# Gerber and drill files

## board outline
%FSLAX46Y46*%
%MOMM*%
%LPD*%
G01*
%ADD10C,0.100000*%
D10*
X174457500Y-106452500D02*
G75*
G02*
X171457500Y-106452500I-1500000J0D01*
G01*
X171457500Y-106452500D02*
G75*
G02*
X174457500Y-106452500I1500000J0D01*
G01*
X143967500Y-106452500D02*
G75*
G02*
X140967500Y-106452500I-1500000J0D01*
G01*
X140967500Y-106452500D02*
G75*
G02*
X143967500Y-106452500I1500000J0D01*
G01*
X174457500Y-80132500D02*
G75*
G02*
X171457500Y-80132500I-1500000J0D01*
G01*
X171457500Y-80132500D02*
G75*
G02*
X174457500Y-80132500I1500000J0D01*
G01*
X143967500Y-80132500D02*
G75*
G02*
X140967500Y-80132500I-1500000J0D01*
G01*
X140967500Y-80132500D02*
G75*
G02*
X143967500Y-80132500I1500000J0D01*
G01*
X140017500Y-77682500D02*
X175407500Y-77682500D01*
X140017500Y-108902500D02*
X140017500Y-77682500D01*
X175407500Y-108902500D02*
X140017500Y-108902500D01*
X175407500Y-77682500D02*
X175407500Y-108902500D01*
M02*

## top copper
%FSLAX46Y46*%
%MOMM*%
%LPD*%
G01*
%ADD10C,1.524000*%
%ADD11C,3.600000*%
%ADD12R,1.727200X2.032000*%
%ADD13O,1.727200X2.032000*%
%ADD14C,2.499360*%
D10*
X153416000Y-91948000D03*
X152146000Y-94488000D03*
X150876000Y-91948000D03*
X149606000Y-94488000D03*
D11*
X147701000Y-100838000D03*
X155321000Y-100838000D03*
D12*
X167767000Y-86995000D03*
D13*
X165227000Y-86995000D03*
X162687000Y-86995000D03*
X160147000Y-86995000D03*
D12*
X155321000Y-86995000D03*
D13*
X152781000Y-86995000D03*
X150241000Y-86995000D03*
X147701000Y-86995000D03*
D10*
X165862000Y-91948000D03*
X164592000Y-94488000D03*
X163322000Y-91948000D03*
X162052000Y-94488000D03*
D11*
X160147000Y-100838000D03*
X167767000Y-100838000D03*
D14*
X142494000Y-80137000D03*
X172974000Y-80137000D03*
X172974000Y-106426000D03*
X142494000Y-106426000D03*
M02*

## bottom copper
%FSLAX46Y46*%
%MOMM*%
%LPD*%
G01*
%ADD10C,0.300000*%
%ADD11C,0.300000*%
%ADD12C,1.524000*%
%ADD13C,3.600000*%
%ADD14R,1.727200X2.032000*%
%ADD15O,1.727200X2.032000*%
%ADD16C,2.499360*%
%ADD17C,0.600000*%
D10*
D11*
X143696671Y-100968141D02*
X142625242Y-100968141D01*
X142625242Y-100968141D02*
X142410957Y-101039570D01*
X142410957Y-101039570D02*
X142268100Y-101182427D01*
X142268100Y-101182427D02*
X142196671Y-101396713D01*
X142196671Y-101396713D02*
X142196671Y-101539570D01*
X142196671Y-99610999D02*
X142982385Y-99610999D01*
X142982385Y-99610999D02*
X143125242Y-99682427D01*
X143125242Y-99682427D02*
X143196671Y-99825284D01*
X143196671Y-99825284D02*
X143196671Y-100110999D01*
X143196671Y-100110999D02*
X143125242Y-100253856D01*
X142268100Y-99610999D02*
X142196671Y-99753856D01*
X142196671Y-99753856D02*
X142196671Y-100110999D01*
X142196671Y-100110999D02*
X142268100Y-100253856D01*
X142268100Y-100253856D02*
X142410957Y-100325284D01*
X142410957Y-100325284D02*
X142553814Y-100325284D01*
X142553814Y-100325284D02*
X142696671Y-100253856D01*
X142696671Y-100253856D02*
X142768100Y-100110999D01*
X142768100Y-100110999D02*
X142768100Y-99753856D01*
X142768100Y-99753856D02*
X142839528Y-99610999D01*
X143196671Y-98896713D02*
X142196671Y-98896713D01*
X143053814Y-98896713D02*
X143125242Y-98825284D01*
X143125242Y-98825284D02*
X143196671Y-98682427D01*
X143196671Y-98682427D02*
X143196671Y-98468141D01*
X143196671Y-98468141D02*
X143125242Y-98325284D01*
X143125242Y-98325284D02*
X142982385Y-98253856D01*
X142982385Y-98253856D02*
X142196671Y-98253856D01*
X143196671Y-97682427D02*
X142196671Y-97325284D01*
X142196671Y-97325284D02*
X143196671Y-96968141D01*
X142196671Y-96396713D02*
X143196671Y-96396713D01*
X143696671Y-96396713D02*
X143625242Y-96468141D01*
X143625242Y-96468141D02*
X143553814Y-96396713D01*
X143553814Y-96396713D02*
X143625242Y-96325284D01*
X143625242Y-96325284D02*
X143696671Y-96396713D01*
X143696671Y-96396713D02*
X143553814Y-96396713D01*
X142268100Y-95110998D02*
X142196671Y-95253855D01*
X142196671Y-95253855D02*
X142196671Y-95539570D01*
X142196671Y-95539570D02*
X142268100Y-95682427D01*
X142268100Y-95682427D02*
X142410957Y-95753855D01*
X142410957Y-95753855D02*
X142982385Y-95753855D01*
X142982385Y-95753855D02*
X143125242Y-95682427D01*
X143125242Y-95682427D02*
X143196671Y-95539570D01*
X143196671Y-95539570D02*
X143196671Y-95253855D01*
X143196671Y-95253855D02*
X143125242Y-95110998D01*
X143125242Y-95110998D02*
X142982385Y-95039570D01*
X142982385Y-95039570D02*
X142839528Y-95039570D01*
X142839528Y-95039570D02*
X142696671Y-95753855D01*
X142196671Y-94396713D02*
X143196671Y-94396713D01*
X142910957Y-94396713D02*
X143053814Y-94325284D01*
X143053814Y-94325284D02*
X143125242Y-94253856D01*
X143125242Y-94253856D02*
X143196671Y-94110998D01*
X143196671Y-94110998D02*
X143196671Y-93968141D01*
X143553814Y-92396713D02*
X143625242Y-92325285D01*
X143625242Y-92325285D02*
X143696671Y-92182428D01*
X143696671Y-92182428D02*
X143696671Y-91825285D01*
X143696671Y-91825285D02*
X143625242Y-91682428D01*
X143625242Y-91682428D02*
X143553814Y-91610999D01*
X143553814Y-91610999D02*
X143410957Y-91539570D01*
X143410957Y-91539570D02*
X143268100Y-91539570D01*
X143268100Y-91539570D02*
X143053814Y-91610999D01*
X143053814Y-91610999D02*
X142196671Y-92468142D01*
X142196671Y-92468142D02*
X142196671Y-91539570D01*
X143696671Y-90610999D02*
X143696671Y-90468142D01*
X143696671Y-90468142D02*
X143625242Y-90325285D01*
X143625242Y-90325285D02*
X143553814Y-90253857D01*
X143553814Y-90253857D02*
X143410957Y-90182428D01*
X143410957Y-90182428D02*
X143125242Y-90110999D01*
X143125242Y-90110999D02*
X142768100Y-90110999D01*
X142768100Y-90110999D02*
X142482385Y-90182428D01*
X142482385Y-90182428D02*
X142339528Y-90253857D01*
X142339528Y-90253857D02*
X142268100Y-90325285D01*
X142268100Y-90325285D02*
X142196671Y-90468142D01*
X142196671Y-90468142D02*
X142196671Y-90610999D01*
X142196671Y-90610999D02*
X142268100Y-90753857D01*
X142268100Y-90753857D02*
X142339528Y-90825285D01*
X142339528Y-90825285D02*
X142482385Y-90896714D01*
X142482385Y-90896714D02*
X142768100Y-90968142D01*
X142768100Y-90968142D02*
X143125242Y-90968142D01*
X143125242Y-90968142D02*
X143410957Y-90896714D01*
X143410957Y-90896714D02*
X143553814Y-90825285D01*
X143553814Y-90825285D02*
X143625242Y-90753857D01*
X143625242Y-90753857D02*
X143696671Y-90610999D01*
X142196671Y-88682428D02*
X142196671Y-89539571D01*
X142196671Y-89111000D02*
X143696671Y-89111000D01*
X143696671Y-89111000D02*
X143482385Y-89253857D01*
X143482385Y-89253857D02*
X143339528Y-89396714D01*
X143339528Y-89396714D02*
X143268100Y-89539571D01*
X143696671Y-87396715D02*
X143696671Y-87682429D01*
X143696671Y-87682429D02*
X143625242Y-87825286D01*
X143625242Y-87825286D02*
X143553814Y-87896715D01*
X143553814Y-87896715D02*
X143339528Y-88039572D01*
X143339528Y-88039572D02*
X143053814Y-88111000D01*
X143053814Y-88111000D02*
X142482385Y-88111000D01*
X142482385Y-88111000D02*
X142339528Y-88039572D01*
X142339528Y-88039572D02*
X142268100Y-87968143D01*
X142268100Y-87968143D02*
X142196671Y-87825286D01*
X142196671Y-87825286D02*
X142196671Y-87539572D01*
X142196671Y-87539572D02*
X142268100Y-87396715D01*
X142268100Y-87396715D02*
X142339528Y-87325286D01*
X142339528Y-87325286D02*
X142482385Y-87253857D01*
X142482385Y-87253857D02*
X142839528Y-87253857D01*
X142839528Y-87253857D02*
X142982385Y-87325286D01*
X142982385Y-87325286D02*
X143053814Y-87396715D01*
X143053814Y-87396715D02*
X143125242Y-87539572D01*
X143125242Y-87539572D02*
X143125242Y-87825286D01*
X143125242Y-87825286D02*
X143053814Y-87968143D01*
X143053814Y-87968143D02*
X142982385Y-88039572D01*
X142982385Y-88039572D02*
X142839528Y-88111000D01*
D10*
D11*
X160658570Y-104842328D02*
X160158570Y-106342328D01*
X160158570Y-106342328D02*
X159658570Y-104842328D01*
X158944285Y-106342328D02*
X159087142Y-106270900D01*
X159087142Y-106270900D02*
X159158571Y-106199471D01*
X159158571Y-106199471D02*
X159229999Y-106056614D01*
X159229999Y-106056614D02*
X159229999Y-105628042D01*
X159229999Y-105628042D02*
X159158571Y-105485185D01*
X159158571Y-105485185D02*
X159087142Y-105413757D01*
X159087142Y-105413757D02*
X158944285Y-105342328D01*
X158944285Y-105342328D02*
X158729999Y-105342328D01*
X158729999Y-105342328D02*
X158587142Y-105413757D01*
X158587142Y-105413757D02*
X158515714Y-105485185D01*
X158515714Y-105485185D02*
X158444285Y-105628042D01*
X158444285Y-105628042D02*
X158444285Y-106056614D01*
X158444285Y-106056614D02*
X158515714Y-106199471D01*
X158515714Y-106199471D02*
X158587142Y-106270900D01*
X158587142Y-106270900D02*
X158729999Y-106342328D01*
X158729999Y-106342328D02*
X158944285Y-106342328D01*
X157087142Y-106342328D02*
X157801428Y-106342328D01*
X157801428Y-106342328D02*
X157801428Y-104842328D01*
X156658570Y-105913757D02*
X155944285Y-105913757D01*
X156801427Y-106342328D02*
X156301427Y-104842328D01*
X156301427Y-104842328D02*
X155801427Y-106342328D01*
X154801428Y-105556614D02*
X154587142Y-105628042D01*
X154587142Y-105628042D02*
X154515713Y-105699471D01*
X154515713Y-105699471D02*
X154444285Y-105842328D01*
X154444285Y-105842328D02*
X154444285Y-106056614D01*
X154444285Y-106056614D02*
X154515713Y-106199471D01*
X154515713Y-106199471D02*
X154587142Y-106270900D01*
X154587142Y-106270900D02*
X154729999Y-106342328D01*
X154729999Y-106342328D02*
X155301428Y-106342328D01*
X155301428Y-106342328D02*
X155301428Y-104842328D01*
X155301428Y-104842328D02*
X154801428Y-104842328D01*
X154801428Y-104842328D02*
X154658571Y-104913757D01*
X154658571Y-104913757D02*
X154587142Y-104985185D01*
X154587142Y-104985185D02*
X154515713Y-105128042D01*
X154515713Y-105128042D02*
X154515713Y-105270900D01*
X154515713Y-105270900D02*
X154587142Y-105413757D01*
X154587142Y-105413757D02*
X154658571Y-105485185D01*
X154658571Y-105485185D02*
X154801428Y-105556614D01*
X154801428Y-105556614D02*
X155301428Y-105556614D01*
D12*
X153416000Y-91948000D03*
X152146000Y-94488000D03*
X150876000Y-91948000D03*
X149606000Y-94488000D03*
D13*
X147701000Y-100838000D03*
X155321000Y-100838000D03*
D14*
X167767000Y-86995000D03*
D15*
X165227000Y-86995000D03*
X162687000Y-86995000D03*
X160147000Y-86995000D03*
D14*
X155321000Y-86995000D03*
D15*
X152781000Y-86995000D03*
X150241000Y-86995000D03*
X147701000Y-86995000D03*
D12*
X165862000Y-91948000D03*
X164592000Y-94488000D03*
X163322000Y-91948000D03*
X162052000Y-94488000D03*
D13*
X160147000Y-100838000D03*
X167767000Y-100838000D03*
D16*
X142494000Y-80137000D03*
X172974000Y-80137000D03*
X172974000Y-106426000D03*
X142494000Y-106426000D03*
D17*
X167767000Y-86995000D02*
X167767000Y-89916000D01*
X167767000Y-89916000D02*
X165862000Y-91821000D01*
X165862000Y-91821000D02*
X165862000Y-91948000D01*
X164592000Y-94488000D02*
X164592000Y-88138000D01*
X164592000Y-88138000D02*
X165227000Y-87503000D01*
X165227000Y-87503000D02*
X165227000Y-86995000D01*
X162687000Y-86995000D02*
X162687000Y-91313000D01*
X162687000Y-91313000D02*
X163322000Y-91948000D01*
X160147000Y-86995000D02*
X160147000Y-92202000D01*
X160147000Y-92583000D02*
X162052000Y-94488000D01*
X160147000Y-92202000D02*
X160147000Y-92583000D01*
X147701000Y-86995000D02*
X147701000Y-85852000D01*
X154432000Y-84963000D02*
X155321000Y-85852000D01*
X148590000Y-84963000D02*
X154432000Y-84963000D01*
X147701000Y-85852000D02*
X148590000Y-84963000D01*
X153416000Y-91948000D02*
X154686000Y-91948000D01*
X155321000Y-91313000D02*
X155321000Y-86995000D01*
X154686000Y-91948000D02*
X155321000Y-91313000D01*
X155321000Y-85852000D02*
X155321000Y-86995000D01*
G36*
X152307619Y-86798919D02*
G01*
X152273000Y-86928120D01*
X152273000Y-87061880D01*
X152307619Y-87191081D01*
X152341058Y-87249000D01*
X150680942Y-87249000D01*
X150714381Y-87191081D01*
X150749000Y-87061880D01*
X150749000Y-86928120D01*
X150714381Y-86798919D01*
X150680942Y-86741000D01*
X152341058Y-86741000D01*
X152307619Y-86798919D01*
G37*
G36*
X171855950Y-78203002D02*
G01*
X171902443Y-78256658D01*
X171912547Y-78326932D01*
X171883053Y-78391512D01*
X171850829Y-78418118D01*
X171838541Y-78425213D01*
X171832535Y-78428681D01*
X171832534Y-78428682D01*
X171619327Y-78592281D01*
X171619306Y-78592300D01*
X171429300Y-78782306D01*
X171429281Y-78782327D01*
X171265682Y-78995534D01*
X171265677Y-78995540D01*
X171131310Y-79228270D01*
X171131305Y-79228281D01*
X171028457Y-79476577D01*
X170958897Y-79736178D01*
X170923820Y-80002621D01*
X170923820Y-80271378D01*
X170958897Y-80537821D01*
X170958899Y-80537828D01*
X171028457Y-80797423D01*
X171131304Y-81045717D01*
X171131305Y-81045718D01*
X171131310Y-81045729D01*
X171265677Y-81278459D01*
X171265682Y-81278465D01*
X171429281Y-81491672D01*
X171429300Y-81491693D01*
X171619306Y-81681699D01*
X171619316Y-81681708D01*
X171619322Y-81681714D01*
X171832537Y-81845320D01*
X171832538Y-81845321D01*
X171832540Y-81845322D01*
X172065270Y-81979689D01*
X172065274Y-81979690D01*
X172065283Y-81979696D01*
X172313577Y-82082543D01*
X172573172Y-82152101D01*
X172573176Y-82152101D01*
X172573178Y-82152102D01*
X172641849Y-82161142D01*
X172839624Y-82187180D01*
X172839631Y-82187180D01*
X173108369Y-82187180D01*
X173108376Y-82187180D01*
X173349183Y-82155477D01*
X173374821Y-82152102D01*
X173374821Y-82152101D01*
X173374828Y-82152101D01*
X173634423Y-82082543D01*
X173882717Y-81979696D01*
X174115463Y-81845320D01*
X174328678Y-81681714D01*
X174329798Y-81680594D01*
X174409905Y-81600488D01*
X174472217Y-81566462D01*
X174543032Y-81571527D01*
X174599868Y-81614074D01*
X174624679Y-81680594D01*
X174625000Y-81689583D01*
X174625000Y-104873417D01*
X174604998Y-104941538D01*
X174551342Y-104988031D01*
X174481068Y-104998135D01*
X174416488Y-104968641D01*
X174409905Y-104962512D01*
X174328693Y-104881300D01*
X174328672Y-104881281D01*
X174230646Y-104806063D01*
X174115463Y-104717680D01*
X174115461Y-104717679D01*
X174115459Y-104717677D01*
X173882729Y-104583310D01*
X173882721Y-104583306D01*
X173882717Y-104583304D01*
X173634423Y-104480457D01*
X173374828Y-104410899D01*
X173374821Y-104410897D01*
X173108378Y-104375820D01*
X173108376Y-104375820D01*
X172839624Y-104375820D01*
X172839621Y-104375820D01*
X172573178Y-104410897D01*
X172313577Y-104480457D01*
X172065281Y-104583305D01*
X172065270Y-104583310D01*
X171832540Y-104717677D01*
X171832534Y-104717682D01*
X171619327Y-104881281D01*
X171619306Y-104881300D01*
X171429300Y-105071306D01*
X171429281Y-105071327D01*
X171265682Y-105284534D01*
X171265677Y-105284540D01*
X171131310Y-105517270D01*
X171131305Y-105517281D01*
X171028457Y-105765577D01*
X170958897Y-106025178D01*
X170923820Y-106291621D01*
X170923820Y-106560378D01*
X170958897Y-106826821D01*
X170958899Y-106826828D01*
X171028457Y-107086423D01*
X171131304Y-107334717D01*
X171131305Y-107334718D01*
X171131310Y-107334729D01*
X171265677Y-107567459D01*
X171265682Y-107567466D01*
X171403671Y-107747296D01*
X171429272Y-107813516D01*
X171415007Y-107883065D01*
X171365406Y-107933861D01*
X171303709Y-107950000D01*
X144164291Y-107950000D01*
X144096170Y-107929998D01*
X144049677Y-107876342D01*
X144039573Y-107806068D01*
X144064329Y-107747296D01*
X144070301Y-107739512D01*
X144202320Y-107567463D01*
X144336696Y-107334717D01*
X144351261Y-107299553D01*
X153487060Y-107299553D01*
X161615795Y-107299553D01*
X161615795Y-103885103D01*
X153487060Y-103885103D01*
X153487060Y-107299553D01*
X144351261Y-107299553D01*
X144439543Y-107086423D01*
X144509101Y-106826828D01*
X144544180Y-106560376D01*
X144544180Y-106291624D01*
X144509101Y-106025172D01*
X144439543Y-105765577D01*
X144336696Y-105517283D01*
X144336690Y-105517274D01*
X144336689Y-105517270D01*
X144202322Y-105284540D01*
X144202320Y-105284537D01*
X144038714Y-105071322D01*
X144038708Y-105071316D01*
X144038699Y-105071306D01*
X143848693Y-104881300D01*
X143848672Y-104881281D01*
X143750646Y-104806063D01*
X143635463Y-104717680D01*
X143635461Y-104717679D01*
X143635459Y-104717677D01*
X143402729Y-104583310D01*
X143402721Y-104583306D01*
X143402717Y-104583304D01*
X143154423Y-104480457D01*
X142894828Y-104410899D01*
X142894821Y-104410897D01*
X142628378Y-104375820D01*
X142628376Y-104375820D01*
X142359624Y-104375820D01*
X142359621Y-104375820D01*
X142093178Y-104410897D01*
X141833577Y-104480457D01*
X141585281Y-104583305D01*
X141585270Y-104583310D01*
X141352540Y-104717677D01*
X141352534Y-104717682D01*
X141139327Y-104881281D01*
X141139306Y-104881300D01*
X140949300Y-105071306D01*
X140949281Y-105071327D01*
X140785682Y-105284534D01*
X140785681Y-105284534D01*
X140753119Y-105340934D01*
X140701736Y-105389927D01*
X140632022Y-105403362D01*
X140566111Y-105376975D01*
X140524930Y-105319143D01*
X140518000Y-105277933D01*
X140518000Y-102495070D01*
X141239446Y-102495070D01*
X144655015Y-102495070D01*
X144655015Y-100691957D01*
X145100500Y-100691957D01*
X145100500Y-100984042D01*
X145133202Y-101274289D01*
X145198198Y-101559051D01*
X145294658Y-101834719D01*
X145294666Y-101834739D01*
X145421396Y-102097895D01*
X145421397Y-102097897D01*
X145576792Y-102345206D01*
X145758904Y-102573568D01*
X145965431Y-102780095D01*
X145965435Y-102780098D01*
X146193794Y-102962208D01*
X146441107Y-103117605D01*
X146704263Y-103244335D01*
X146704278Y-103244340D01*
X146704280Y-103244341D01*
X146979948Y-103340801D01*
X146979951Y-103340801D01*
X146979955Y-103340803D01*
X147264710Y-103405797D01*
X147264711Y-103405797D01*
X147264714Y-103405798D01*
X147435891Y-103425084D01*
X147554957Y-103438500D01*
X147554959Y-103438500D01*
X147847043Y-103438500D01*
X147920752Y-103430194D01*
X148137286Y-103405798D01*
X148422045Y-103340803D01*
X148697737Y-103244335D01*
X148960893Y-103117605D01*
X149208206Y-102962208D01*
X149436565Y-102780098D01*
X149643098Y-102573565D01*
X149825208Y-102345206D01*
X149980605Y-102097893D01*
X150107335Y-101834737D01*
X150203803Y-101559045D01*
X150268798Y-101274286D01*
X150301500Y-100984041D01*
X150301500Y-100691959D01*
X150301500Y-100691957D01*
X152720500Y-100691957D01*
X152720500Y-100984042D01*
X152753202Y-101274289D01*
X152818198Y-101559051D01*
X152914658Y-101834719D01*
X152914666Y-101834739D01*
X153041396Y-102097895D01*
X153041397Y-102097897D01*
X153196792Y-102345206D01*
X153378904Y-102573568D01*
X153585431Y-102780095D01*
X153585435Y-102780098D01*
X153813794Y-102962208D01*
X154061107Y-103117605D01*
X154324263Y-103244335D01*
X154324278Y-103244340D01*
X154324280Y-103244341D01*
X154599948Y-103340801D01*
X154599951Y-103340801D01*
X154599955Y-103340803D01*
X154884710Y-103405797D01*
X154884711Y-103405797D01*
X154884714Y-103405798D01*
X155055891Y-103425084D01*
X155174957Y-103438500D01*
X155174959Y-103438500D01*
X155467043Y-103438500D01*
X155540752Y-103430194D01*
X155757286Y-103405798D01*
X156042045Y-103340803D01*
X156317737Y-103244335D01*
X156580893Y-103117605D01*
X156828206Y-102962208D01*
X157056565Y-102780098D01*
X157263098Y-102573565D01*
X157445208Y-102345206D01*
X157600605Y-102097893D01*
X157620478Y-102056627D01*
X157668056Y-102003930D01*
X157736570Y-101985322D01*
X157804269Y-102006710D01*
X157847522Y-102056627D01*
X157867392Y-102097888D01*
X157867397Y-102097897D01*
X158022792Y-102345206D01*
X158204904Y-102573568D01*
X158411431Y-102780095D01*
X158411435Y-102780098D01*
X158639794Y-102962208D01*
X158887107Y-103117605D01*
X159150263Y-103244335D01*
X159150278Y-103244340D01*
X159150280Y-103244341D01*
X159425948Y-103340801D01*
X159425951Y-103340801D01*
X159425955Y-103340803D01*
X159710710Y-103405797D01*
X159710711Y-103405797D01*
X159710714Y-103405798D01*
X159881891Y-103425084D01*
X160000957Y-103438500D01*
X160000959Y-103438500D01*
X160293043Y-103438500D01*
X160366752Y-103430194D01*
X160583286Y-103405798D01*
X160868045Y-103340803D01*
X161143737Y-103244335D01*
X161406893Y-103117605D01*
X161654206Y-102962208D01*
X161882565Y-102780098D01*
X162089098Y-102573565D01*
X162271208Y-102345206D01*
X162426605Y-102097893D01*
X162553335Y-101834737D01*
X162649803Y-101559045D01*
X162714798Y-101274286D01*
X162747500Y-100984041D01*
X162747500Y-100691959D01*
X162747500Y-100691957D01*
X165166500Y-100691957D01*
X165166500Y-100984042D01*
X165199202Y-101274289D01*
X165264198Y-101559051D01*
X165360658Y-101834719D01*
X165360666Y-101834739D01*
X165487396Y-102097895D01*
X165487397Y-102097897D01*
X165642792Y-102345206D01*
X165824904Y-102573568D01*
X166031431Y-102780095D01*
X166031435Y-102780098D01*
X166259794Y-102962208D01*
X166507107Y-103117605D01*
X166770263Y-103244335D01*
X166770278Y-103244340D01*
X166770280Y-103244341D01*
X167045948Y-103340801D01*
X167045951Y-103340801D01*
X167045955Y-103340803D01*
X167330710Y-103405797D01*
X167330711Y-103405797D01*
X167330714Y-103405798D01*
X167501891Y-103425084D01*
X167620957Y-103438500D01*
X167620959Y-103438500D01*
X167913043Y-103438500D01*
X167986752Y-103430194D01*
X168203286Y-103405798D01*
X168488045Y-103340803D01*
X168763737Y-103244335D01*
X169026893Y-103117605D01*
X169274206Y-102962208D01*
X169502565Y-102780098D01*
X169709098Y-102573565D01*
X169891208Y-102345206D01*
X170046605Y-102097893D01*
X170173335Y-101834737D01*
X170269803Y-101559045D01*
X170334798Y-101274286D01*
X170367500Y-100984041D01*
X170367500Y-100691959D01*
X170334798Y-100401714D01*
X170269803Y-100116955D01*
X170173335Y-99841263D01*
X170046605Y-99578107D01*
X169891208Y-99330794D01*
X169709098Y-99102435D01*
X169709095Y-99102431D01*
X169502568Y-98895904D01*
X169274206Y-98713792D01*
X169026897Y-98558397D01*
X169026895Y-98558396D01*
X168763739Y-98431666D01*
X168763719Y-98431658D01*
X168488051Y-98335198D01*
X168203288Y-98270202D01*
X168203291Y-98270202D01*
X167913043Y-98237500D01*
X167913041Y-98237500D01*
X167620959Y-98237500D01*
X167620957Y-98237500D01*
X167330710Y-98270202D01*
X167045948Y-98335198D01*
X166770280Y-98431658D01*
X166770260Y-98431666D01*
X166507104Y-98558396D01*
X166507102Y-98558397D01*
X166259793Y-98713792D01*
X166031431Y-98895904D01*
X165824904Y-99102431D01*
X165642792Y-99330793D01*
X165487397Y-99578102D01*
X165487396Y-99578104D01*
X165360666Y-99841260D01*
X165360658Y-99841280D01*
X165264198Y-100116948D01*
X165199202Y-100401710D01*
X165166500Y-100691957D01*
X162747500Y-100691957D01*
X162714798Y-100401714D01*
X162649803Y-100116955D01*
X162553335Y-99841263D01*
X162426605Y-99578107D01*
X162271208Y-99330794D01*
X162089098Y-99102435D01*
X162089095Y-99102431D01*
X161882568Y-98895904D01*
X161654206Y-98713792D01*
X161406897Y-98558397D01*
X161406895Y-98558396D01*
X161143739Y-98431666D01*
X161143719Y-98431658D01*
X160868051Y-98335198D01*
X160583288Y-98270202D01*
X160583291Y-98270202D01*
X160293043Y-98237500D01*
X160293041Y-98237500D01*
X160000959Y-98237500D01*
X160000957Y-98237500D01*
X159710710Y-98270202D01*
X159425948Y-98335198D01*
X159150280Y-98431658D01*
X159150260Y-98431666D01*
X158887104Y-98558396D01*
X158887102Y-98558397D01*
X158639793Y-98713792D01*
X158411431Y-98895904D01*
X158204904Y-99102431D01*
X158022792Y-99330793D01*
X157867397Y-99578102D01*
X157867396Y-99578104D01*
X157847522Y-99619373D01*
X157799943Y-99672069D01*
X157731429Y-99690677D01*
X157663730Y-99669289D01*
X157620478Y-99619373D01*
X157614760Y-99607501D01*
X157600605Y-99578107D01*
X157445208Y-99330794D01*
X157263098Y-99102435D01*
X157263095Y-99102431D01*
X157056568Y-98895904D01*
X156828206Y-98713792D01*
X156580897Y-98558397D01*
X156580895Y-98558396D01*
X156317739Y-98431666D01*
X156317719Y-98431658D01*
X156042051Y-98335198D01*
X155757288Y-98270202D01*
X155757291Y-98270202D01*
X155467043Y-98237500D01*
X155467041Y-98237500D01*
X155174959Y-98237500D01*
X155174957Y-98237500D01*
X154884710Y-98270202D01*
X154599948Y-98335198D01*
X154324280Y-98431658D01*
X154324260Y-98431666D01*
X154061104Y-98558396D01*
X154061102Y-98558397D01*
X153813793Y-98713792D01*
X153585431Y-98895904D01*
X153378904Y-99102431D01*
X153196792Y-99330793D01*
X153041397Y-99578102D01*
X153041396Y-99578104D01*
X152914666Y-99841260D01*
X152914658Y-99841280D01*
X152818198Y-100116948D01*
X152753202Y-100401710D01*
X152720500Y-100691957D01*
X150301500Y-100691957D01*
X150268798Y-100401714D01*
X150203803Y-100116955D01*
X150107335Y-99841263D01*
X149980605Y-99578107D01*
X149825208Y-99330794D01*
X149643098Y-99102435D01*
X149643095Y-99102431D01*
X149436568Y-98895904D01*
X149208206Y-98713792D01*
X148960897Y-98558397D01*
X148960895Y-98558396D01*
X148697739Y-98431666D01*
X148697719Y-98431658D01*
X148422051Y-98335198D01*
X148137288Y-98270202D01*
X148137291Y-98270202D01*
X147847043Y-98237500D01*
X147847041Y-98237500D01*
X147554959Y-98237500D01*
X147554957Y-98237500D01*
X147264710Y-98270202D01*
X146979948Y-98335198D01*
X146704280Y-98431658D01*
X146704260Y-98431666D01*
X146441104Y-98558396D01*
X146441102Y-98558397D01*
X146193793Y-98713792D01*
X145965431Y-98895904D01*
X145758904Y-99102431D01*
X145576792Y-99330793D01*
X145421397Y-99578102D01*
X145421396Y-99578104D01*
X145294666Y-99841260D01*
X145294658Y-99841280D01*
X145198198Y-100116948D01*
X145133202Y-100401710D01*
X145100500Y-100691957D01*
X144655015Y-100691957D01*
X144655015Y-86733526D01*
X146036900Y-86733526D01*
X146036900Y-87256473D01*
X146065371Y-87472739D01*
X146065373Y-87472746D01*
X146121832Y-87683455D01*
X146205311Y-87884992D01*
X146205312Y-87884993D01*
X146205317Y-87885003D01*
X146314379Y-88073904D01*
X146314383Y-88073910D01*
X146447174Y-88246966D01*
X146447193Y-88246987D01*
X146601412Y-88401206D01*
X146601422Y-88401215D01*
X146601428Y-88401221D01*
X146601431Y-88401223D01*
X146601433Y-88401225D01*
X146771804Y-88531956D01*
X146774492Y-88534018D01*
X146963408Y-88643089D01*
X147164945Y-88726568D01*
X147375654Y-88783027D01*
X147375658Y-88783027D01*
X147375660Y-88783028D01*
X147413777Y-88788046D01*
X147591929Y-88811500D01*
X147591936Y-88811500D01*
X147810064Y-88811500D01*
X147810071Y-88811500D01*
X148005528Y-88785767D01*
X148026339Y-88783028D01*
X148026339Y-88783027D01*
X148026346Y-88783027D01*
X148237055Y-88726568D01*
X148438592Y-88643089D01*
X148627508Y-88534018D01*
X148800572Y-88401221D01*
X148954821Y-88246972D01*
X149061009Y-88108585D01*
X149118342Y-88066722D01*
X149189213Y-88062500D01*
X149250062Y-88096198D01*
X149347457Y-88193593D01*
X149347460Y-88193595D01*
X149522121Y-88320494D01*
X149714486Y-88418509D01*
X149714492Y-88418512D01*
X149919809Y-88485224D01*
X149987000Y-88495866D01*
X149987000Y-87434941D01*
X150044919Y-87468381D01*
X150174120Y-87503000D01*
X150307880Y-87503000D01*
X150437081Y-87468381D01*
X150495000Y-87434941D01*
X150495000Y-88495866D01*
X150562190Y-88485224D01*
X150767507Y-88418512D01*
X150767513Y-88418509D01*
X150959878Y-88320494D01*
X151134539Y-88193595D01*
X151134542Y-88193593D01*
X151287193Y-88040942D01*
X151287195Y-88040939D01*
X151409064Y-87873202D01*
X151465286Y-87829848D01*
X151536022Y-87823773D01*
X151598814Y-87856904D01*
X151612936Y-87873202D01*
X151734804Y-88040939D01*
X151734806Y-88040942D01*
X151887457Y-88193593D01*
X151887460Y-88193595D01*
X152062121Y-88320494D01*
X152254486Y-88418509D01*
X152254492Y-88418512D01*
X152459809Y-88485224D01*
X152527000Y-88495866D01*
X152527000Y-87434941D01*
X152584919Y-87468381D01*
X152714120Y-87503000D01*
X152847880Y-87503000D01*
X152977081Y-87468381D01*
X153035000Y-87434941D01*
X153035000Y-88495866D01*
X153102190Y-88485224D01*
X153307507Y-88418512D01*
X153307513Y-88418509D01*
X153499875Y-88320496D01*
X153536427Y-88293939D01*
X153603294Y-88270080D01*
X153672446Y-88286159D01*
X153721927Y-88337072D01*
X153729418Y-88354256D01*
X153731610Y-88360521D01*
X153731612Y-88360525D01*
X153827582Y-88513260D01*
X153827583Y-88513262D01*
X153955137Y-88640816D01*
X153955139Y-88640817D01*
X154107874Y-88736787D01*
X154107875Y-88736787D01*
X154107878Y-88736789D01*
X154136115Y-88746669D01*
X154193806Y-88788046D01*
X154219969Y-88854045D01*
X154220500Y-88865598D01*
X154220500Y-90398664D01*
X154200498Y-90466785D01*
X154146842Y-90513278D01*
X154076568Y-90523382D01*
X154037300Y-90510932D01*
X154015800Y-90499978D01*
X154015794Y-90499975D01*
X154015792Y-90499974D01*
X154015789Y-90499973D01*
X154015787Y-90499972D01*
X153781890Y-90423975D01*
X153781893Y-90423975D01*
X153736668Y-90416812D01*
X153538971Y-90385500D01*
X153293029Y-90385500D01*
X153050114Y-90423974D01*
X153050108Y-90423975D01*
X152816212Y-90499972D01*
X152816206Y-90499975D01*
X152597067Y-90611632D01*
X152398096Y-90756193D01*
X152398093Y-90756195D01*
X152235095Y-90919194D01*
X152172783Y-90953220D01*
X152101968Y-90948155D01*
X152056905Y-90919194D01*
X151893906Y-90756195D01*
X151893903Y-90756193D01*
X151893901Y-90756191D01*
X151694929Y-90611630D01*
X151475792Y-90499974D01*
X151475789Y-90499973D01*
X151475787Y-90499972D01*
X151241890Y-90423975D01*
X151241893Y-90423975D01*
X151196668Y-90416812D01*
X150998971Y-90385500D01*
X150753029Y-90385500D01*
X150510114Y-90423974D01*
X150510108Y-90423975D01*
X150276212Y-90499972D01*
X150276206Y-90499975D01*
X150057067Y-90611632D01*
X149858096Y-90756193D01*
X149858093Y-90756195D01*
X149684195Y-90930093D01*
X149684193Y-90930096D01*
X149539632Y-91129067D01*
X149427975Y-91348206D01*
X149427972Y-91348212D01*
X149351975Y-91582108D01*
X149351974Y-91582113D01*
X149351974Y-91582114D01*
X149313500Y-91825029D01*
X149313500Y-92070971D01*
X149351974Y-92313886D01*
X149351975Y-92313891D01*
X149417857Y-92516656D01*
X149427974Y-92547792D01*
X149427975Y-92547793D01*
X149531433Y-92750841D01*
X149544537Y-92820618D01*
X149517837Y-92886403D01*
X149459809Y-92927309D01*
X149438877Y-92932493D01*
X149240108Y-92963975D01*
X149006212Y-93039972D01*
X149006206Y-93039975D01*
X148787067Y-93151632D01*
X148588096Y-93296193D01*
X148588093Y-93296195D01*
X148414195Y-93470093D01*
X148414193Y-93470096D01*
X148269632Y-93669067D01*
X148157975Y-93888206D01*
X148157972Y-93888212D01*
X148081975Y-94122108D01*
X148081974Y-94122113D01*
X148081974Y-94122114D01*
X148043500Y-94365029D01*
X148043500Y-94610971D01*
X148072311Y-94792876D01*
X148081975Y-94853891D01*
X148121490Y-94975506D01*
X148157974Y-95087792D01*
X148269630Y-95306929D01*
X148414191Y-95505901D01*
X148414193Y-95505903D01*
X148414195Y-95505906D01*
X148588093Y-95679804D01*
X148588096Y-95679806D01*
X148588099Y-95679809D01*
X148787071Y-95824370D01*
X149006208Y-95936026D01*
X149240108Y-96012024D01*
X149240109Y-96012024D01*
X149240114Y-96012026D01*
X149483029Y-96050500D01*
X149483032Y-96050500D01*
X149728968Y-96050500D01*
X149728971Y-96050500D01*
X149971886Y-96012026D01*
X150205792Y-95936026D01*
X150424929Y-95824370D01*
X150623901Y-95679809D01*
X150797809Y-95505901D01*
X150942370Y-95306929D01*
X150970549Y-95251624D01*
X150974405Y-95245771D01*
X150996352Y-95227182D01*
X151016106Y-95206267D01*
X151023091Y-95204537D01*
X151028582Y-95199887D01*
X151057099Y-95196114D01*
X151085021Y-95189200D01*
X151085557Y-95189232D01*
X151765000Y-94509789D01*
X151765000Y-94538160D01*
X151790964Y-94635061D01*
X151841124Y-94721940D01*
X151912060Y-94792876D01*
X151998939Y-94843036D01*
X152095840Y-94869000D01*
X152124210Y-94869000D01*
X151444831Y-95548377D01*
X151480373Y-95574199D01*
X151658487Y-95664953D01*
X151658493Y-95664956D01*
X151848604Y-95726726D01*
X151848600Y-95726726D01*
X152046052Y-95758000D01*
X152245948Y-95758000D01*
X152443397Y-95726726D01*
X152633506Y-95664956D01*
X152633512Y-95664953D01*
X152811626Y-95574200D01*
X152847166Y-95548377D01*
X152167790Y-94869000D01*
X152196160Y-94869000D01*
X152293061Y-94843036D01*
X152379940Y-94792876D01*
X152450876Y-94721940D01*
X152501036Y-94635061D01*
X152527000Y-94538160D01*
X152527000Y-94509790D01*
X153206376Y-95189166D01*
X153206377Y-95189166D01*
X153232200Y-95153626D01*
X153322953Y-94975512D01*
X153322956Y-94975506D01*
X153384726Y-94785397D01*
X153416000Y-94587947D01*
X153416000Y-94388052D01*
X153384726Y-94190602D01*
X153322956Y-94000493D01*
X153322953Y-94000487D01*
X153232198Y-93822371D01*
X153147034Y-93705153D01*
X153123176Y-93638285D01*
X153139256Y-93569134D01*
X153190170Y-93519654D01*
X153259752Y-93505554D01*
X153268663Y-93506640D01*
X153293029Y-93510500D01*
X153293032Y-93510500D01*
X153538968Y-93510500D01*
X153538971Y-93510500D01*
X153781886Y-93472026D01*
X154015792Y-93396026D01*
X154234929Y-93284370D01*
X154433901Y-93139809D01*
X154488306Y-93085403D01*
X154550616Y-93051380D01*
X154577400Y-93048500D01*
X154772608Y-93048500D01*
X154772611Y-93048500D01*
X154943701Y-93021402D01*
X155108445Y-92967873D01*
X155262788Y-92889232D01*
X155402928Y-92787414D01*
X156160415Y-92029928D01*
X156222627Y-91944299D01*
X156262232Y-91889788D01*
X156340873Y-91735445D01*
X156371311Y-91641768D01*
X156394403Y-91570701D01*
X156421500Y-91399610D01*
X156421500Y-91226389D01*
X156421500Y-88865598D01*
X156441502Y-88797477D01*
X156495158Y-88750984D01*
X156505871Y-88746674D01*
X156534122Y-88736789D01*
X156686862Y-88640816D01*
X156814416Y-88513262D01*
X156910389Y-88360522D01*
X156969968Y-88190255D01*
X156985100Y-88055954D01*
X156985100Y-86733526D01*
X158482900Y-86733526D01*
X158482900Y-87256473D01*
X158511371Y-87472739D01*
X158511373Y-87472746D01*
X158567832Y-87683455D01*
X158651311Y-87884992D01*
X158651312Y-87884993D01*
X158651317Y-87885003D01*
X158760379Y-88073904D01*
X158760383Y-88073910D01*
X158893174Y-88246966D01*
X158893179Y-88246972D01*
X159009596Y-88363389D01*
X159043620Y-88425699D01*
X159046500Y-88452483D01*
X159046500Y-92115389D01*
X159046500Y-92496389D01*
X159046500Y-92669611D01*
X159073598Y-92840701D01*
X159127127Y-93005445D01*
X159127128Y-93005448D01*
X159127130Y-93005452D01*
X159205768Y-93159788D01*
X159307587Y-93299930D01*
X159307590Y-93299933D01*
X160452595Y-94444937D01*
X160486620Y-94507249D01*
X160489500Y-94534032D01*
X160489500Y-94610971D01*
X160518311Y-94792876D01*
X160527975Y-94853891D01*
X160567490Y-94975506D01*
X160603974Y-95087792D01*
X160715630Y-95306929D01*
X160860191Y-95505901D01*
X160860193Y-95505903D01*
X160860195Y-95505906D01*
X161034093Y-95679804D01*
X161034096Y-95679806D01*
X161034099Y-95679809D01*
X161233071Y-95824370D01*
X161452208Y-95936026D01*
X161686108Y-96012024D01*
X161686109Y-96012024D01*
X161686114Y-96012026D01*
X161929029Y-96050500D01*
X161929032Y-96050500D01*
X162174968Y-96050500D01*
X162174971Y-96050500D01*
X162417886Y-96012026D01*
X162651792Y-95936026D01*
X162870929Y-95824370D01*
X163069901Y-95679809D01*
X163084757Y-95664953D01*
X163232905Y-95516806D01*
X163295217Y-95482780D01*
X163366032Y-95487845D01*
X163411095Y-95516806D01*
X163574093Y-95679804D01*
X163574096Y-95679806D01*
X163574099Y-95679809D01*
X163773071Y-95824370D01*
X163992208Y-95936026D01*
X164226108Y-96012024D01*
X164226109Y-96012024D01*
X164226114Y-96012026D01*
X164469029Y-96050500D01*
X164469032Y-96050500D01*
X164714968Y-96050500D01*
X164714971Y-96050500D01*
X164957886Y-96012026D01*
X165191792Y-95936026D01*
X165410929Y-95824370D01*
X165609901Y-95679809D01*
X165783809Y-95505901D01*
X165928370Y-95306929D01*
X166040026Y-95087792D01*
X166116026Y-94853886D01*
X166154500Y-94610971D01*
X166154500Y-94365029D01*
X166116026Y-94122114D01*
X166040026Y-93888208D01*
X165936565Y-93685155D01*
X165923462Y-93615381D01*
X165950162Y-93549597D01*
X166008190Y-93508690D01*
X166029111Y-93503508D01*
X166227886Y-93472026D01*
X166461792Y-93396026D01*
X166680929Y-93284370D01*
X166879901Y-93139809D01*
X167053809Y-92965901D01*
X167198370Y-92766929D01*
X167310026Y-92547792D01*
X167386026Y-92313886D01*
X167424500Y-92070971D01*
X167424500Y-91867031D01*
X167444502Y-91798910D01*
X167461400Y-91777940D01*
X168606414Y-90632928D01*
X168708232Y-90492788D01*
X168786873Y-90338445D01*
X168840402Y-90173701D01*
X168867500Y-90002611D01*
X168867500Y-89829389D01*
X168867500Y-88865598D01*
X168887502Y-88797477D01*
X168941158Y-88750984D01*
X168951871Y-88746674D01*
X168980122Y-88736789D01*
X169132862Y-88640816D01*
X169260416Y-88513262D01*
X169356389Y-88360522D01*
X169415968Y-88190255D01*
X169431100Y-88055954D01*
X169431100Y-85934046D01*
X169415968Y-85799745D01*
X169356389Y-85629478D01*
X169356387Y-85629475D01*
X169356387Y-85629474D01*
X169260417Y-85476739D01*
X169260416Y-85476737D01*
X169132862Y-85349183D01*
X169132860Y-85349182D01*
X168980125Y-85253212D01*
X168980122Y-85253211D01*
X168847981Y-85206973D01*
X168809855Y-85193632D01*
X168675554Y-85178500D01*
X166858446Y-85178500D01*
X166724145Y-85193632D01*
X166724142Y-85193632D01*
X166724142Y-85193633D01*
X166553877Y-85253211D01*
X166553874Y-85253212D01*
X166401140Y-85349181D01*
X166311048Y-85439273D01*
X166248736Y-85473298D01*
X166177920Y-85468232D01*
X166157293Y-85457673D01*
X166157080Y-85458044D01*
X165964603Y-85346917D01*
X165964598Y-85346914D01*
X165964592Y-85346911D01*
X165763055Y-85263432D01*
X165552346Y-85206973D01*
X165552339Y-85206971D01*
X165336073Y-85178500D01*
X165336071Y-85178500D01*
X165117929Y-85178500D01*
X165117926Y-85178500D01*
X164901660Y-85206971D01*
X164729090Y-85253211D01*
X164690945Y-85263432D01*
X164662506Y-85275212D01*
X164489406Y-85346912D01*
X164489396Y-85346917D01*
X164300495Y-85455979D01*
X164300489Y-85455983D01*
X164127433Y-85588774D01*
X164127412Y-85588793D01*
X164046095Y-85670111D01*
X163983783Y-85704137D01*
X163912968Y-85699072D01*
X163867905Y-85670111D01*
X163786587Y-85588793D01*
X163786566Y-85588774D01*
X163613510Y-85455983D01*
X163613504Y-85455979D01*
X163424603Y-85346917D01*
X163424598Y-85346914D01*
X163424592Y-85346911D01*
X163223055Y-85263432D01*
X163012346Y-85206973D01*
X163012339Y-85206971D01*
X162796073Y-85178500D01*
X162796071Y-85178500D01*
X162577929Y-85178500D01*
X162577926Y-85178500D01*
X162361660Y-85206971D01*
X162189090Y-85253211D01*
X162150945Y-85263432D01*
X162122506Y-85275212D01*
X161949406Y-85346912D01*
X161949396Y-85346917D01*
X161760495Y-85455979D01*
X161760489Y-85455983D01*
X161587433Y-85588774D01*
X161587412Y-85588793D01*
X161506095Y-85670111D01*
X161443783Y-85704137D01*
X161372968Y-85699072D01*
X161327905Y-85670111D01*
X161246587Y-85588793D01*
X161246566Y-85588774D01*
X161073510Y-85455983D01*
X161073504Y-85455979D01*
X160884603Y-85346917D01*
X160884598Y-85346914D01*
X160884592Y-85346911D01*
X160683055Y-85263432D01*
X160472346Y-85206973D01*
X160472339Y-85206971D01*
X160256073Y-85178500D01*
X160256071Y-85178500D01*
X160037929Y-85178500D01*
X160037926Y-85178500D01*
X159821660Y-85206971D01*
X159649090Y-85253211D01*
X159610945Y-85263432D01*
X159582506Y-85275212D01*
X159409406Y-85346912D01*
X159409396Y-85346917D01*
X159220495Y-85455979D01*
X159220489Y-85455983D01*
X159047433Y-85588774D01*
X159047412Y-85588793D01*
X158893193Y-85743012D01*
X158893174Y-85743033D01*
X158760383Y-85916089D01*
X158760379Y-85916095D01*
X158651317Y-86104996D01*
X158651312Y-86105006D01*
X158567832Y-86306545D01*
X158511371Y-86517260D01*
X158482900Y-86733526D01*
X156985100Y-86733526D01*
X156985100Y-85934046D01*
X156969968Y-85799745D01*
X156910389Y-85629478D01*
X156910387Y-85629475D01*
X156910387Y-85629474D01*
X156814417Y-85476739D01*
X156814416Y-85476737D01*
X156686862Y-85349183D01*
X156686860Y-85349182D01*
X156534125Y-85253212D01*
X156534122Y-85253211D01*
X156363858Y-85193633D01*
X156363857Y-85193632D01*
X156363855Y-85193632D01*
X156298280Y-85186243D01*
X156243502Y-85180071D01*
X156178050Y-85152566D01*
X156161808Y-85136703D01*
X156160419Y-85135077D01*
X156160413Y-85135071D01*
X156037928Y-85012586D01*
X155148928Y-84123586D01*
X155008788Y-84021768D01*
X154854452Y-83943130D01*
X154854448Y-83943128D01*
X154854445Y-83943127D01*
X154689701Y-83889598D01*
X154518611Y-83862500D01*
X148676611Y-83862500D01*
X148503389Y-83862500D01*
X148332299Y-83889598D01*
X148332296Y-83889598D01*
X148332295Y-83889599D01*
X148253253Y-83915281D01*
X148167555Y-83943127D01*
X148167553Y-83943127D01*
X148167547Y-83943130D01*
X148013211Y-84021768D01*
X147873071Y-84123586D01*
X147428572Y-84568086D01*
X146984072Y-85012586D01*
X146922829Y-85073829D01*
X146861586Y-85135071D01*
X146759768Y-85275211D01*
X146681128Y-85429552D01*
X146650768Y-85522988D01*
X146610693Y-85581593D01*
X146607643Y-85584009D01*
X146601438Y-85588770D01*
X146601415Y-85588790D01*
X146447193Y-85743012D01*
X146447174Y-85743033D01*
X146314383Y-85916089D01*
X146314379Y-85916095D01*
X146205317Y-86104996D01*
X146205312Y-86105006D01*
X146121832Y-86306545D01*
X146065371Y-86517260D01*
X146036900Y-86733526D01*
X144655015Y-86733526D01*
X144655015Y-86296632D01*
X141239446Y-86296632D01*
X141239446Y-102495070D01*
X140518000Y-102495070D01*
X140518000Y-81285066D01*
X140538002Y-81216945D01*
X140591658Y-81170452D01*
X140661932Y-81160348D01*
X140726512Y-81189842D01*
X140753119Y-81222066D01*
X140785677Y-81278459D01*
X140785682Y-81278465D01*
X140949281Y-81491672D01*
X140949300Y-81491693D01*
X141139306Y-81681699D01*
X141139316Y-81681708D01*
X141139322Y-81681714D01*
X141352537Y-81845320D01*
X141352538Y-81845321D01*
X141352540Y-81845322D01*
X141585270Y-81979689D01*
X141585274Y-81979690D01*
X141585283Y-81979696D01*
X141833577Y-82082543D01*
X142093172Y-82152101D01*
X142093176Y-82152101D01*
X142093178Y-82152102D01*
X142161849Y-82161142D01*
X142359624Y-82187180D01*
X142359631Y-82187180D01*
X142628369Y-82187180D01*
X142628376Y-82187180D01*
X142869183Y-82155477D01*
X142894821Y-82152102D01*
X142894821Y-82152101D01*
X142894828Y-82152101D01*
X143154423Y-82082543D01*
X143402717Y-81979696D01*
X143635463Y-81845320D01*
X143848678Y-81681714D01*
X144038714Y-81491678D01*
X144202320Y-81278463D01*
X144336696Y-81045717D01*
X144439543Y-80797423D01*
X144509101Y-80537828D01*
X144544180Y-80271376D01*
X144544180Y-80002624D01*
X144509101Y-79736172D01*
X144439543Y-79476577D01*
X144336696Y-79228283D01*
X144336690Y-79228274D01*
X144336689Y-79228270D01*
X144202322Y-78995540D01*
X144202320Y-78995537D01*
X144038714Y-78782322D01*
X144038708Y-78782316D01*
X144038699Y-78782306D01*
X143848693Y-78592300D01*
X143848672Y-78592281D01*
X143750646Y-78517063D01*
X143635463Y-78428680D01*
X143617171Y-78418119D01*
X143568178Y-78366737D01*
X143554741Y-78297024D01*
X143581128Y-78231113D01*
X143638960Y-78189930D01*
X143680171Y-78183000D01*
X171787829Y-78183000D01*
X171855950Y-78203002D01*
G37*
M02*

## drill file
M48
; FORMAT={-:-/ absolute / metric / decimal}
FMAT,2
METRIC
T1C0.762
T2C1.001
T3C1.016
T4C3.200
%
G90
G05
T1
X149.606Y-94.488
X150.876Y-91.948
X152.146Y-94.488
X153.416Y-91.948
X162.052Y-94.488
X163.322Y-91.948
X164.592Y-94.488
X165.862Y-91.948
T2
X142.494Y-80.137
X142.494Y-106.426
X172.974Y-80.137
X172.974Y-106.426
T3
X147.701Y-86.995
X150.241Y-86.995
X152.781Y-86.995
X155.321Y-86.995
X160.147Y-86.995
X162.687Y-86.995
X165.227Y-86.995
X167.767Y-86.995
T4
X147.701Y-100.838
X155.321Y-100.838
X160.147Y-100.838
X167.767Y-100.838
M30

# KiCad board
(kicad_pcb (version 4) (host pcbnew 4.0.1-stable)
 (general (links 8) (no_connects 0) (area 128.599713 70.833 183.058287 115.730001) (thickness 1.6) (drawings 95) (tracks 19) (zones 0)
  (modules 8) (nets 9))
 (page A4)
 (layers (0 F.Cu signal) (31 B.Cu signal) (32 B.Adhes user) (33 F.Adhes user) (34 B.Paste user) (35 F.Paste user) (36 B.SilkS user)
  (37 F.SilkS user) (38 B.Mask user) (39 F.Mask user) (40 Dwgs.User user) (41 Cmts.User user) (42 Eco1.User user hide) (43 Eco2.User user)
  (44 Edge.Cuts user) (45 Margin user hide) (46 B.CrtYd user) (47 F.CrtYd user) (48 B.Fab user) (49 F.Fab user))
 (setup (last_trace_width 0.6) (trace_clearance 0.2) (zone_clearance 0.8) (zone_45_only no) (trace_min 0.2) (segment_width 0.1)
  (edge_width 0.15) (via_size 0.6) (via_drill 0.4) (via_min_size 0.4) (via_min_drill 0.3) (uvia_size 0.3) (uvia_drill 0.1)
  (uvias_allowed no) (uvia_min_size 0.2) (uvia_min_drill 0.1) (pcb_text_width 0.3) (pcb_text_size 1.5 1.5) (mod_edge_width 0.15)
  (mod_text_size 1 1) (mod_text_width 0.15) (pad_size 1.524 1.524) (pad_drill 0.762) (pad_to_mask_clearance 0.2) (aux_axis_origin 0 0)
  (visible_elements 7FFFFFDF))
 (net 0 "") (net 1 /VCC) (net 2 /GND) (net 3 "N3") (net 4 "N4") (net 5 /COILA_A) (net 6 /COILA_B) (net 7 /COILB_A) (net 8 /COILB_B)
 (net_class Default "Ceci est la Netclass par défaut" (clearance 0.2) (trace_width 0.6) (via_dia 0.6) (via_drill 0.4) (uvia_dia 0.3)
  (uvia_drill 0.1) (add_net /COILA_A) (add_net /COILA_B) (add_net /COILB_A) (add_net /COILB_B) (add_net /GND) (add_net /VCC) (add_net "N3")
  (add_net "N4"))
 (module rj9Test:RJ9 (layer F.Cu) (at 151.511 100.838)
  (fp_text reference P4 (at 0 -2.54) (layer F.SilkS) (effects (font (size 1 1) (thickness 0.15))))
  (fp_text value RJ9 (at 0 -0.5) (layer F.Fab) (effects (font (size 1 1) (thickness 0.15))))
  (pad 1 thru_hole circle (at 1.905 -8.89) (size 1.524 1.524) (drill 0.762) (layers *.Cu *.Mask F.SilkS) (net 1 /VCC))
  (pad 2 thru_hole circle (at 0.635 -6.35) (size 1.524 1.524) (drill 0.762) (layers *.Cu *.Mask F.SilkS) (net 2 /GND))
  (pad 3 thru_hole circle (at -0.635 -8.89) (size 1.524 1.524) (drill 0.762) (layers *.Cu *.Mask F.SilkS) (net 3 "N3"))
  (pad 4 thru_hole circle (at -1.905 -6.35) (size 1.524 1.524) (drill 0.762) (layers *.Cu *.Mask F.SilkS) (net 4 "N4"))
  (pad "" thru_hole circle (at -3.81 0) (size 3.6 3.6) (drill 3.2) (layers *.Cu *.Mask F.SilkS))
  (pad "" thru_hole circle (at 3.81 0) (size 3.6 3.6) (drill 3.2) (layers *.Cu *.Mask F.SilkS)))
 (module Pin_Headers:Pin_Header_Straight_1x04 (layer F.Cu) (at 167.767 86.995 270)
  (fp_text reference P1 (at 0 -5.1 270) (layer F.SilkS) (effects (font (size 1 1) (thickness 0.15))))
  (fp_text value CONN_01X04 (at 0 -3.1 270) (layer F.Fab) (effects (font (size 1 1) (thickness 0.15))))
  (pad 1 thru_hole rect (at 0 0 270) (size 2.032 1.7272) (drill 1.016) (layers *.Cu *.Mask F.SilkS) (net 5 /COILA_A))
  (pad 2 thru_hole oval (at 0 2.54 270) (size 2.032 1.7272) (drill 1.016) (layers *.Cu *.Mask F.SilkS) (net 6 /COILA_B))
  (pad 3 thru_hole oval (at 0 5.08 270) (size 2.032 1.7272) (drill 1.016) (layers *.Cu *.Mask F.SilkS) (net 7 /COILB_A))
  (pad 4 thru_hole oval (at 0 7.62 270) (size 2.032 1.7272) (drill 1.016) (layers *.Cu *.Mask F.SilkS) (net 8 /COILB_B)))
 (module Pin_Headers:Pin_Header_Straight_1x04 (layer F.Cu) (at 155.321 86.995 270)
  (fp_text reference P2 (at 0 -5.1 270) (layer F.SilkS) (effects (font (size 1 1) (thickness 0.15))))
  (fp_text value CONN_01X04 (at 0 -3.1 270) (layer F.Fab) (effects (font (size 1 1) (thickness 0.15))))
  (pad 1 thru_hole rect (at 0 0 270) (size 2.032 1.7272) (drill 1.016) (layers *.Cu *.Mask F.SilkS) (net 1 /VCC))
  (pad 2 thru_hole oval (at 0 2.54 270) (size 2.032 1.7272) (drill 1.016) (layers *.Cu *.Mask F.SilkS) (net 2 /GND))
  (pad 3 thru_hole oval (at 0 5.08 270) (size 2.032 1.7272) (drill 1.016) (layers *.Cu *.Mask F.SilkS) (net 2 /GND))
  (pad 4 thru_hole oval (at 0 7.62 270) (size 2.032 1.7272) (drill 1.016) (layers *.Cu *.Mask F.SilkS) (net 1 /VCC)))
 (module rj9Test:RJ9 (layer F.Cu) (at 163.957 100.838)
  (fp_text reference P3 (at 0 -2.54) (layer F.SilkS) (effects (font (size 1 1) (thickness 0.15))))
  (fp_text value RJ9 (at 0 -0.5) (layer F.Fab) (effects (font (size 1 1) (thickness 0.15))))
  (pad 1 thru_hole circle (at 1.905 -8.89) (size 1.524 1.524) (drill 0.762) (layers *.Cu *.Mask F.SilkS) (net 5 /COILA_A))
  (pad 2 thru_hole circle (at 0.635 -6.35) (size 1.524 1.524) (drill 0.762) (layers *.Cu *.Mask F.SilkS) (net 6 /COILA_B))
  (pad 3 thru_hole circle (at -0.635 -8.89) (size 1.524 1.524) (drill 0.762) (layers *.Cu *.Mask F.SilkS) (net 7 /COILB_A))
  (pad 4 thru_hole circle (at -1.905 -6.35) (size 1.524 1.524) (drill 0.762) (layers *.Cu *.Mask F.SilkS) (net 8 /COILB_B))
  (pad "" thru_hole circle (at -3.81 0) (size 3.6 3.6) (drill 3.2) (layers *.Cu *.Mask F.SilkS))
  (pad "" thru_hole circle (at 3.81 0) (size 3.6 3.6) (drill 3.2) (layers *.Cu *.Mask F.SilkS)))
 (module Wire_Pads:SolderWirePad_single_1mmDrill (layer F.Cu) (at 142.494 80.137)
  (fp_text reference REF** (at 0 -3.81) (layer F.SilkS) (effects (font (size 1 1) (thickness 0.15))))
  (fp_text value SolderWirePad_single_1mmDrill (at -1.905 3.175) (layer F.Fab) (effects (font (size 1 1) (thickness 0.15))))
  (pad 1 thru_hole circle (at 0 0) (size 2.49936 2.49936) (drill 1.00076) (layers *.Cu *.Mask F.SilkS)))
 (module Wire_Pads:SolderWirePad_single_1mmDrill (layer F.Cu) (at 172.974 80.137)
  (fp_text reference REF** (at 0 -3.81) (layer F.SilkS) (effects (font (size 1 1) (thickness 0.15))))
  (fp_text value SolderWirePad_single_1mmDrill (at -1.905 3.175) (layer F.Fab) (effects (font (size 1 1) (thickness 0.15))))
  (pad 1 thru_hole circle (at 0 0) (size 2.49936 2.49936) (drill 1.00076) (layers *.Cu *.Mask F.SilkS)))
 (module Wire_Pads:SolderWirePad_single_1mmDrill (layer F.Cu) (at 172.974 106.426)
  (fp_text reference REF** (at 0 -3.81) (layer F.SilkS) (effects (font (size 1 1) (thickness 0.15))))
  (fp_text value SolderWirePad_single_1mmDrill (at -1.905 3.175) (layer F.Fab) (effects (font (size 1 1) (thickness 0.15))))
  (pad 1 thru_hole circle (at 0 0) (size 2.49936 2.49936) (drill 1.00076) (layers *.Cu *.Mask F.SilkS)))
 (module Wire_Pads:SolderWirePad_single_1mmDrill (layer F.Cu) (at 142.494 106.426)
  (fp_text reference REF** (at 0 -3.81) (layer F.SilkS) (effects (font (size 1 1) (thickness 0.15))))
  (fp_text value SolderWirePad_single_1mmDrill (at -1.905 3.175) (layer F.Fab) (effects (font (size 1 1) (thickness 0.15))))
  (pad 1 thru_hole circle (at 0 0) (size 2.49936 2.49936) (drill 1.00076) (layers *.Cu *.Mask F.SilkS)))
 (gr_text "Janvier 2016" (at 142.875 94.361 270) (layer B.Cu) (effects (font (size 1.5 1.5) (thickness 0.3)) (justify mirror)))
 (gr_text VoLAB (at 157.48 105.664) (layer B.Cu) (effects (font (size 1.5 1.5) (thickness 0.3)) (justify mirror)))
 (gr_circle (center 172.9575 106.4525) (end 172.9575 104.9525) (layer Edge.Cuts) (width 0.1))
 (gr_circle (center 142.4675 106.4525) (end 142.4675 104.9525) (layer Edge.Cuts) (width 0.1))
 (gr_circle (center 172.9575 80.1325) (end 172.9575 78.6325) (layer Edge.Cuts) (width 0.1))
 (gr_circle (center 142.4675 80.1325) (end 142.4675 78.6325) (layer Edge.Cuts) (width 0.1))
 (gr_line (start 140.0175 77.6825) (end 175.4075 77.6825) (layer Edge.Cuts) (width 0.1))
 (gr_line (start 140.0175 108.9025) (end 140.0175 77.6825) (layer Edge.Cuts) (width 0.1))
 (gr_line (start 175.4075 108.9025) (end 140.0175 108.9025) (layer Edge.Cuts) (width 0.1))
 (gr_line (start 175.4075 77.6825) (end 175.4075 108.9025) (layer Edge.Cuts) (width 0.1))
 (segment (start 167.767 86.995) (end 167.767 89.916) (width 0.6) (layer B.Cu) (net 5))
 (segment (start 167.767 89.916) (end 165.862 91.821) (width 0.6) (layer B.Cu) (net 5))
 (segment (start 165.862 91.821) (end 165.862 91.948) (width 0.6) (layer B.Cu) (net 5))
 (segment (start 164.592 94.488) (end 164.592 88.138) (width 0.6) (layer B.Cu) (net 6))
 (segment (start 164.592 88.138) (end 165.227 87.503) (width 0.6) (layer B.Cu) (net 6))
 (segment (start 165.227 87.503) (end 165.227 86.995) (width 0.6) (layer B.Cu) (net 6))
 (segment (start 162.687 86.995) (end 162.687 91.313) (width 0.6) (layer B.Cu) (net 7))
 (segment (start 162.687 91.313) (end 163.322 91.948) (width 0.6) (layer B.Cu) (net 7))
 (segment (start 160.147 86.995) (end 160.147 92.202) (width 0.6) (layer B.Cu) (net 8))
 (segment (start 160.147 92.583) (end 162.052 94.488) (width 0.6) (layer B.Cu) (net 8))
 (segment (start 160.147 92.202) (end 160.147 92.583) (width 0.6) (layer B.Cu) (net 8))
 (segment (start 147.701 86.995) (end 147.701 85.852) (width 0.6) (layer B.Cu) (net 1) (status 400000))
 (segment (start 154.432 84.963) (end 155.321 85.852) (width 0.6) (layer B.Cu) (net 1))
 (segment (start 148.59 84.963) (end 154.432 84.963) (width 0.6) (layer B.Cu) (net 1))
 (segment (start 147.701 85.852) (end 148.59 84.963) (width 0.6) (layer B.Cu) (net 1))
 (segment (start 153.416 91.948) (end 154.686 91.948) (width 0.6) (layer B.Cu) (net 1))
 (segment (start 155.321 91.313) (end 155.321 86.995) (width 0.6) (layer B.Cu) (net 1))
 (segment (start 154.686 91.948) (end 155.321 91.313) (width 0.6) (layer B.Cu) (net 1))
 (segment (start 155.321 85.852) (end 155.321 86.995) (width 0.6) (layer B.Cu) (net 1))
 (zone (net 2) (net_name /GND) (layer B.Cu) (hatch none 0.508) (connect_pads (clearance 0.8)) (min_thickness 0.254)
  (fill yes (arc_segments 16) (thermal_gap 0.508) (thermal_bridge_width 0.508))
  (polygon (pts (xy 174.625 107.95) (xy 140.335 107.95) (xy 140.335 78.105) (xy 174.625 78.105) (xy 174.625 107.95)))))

